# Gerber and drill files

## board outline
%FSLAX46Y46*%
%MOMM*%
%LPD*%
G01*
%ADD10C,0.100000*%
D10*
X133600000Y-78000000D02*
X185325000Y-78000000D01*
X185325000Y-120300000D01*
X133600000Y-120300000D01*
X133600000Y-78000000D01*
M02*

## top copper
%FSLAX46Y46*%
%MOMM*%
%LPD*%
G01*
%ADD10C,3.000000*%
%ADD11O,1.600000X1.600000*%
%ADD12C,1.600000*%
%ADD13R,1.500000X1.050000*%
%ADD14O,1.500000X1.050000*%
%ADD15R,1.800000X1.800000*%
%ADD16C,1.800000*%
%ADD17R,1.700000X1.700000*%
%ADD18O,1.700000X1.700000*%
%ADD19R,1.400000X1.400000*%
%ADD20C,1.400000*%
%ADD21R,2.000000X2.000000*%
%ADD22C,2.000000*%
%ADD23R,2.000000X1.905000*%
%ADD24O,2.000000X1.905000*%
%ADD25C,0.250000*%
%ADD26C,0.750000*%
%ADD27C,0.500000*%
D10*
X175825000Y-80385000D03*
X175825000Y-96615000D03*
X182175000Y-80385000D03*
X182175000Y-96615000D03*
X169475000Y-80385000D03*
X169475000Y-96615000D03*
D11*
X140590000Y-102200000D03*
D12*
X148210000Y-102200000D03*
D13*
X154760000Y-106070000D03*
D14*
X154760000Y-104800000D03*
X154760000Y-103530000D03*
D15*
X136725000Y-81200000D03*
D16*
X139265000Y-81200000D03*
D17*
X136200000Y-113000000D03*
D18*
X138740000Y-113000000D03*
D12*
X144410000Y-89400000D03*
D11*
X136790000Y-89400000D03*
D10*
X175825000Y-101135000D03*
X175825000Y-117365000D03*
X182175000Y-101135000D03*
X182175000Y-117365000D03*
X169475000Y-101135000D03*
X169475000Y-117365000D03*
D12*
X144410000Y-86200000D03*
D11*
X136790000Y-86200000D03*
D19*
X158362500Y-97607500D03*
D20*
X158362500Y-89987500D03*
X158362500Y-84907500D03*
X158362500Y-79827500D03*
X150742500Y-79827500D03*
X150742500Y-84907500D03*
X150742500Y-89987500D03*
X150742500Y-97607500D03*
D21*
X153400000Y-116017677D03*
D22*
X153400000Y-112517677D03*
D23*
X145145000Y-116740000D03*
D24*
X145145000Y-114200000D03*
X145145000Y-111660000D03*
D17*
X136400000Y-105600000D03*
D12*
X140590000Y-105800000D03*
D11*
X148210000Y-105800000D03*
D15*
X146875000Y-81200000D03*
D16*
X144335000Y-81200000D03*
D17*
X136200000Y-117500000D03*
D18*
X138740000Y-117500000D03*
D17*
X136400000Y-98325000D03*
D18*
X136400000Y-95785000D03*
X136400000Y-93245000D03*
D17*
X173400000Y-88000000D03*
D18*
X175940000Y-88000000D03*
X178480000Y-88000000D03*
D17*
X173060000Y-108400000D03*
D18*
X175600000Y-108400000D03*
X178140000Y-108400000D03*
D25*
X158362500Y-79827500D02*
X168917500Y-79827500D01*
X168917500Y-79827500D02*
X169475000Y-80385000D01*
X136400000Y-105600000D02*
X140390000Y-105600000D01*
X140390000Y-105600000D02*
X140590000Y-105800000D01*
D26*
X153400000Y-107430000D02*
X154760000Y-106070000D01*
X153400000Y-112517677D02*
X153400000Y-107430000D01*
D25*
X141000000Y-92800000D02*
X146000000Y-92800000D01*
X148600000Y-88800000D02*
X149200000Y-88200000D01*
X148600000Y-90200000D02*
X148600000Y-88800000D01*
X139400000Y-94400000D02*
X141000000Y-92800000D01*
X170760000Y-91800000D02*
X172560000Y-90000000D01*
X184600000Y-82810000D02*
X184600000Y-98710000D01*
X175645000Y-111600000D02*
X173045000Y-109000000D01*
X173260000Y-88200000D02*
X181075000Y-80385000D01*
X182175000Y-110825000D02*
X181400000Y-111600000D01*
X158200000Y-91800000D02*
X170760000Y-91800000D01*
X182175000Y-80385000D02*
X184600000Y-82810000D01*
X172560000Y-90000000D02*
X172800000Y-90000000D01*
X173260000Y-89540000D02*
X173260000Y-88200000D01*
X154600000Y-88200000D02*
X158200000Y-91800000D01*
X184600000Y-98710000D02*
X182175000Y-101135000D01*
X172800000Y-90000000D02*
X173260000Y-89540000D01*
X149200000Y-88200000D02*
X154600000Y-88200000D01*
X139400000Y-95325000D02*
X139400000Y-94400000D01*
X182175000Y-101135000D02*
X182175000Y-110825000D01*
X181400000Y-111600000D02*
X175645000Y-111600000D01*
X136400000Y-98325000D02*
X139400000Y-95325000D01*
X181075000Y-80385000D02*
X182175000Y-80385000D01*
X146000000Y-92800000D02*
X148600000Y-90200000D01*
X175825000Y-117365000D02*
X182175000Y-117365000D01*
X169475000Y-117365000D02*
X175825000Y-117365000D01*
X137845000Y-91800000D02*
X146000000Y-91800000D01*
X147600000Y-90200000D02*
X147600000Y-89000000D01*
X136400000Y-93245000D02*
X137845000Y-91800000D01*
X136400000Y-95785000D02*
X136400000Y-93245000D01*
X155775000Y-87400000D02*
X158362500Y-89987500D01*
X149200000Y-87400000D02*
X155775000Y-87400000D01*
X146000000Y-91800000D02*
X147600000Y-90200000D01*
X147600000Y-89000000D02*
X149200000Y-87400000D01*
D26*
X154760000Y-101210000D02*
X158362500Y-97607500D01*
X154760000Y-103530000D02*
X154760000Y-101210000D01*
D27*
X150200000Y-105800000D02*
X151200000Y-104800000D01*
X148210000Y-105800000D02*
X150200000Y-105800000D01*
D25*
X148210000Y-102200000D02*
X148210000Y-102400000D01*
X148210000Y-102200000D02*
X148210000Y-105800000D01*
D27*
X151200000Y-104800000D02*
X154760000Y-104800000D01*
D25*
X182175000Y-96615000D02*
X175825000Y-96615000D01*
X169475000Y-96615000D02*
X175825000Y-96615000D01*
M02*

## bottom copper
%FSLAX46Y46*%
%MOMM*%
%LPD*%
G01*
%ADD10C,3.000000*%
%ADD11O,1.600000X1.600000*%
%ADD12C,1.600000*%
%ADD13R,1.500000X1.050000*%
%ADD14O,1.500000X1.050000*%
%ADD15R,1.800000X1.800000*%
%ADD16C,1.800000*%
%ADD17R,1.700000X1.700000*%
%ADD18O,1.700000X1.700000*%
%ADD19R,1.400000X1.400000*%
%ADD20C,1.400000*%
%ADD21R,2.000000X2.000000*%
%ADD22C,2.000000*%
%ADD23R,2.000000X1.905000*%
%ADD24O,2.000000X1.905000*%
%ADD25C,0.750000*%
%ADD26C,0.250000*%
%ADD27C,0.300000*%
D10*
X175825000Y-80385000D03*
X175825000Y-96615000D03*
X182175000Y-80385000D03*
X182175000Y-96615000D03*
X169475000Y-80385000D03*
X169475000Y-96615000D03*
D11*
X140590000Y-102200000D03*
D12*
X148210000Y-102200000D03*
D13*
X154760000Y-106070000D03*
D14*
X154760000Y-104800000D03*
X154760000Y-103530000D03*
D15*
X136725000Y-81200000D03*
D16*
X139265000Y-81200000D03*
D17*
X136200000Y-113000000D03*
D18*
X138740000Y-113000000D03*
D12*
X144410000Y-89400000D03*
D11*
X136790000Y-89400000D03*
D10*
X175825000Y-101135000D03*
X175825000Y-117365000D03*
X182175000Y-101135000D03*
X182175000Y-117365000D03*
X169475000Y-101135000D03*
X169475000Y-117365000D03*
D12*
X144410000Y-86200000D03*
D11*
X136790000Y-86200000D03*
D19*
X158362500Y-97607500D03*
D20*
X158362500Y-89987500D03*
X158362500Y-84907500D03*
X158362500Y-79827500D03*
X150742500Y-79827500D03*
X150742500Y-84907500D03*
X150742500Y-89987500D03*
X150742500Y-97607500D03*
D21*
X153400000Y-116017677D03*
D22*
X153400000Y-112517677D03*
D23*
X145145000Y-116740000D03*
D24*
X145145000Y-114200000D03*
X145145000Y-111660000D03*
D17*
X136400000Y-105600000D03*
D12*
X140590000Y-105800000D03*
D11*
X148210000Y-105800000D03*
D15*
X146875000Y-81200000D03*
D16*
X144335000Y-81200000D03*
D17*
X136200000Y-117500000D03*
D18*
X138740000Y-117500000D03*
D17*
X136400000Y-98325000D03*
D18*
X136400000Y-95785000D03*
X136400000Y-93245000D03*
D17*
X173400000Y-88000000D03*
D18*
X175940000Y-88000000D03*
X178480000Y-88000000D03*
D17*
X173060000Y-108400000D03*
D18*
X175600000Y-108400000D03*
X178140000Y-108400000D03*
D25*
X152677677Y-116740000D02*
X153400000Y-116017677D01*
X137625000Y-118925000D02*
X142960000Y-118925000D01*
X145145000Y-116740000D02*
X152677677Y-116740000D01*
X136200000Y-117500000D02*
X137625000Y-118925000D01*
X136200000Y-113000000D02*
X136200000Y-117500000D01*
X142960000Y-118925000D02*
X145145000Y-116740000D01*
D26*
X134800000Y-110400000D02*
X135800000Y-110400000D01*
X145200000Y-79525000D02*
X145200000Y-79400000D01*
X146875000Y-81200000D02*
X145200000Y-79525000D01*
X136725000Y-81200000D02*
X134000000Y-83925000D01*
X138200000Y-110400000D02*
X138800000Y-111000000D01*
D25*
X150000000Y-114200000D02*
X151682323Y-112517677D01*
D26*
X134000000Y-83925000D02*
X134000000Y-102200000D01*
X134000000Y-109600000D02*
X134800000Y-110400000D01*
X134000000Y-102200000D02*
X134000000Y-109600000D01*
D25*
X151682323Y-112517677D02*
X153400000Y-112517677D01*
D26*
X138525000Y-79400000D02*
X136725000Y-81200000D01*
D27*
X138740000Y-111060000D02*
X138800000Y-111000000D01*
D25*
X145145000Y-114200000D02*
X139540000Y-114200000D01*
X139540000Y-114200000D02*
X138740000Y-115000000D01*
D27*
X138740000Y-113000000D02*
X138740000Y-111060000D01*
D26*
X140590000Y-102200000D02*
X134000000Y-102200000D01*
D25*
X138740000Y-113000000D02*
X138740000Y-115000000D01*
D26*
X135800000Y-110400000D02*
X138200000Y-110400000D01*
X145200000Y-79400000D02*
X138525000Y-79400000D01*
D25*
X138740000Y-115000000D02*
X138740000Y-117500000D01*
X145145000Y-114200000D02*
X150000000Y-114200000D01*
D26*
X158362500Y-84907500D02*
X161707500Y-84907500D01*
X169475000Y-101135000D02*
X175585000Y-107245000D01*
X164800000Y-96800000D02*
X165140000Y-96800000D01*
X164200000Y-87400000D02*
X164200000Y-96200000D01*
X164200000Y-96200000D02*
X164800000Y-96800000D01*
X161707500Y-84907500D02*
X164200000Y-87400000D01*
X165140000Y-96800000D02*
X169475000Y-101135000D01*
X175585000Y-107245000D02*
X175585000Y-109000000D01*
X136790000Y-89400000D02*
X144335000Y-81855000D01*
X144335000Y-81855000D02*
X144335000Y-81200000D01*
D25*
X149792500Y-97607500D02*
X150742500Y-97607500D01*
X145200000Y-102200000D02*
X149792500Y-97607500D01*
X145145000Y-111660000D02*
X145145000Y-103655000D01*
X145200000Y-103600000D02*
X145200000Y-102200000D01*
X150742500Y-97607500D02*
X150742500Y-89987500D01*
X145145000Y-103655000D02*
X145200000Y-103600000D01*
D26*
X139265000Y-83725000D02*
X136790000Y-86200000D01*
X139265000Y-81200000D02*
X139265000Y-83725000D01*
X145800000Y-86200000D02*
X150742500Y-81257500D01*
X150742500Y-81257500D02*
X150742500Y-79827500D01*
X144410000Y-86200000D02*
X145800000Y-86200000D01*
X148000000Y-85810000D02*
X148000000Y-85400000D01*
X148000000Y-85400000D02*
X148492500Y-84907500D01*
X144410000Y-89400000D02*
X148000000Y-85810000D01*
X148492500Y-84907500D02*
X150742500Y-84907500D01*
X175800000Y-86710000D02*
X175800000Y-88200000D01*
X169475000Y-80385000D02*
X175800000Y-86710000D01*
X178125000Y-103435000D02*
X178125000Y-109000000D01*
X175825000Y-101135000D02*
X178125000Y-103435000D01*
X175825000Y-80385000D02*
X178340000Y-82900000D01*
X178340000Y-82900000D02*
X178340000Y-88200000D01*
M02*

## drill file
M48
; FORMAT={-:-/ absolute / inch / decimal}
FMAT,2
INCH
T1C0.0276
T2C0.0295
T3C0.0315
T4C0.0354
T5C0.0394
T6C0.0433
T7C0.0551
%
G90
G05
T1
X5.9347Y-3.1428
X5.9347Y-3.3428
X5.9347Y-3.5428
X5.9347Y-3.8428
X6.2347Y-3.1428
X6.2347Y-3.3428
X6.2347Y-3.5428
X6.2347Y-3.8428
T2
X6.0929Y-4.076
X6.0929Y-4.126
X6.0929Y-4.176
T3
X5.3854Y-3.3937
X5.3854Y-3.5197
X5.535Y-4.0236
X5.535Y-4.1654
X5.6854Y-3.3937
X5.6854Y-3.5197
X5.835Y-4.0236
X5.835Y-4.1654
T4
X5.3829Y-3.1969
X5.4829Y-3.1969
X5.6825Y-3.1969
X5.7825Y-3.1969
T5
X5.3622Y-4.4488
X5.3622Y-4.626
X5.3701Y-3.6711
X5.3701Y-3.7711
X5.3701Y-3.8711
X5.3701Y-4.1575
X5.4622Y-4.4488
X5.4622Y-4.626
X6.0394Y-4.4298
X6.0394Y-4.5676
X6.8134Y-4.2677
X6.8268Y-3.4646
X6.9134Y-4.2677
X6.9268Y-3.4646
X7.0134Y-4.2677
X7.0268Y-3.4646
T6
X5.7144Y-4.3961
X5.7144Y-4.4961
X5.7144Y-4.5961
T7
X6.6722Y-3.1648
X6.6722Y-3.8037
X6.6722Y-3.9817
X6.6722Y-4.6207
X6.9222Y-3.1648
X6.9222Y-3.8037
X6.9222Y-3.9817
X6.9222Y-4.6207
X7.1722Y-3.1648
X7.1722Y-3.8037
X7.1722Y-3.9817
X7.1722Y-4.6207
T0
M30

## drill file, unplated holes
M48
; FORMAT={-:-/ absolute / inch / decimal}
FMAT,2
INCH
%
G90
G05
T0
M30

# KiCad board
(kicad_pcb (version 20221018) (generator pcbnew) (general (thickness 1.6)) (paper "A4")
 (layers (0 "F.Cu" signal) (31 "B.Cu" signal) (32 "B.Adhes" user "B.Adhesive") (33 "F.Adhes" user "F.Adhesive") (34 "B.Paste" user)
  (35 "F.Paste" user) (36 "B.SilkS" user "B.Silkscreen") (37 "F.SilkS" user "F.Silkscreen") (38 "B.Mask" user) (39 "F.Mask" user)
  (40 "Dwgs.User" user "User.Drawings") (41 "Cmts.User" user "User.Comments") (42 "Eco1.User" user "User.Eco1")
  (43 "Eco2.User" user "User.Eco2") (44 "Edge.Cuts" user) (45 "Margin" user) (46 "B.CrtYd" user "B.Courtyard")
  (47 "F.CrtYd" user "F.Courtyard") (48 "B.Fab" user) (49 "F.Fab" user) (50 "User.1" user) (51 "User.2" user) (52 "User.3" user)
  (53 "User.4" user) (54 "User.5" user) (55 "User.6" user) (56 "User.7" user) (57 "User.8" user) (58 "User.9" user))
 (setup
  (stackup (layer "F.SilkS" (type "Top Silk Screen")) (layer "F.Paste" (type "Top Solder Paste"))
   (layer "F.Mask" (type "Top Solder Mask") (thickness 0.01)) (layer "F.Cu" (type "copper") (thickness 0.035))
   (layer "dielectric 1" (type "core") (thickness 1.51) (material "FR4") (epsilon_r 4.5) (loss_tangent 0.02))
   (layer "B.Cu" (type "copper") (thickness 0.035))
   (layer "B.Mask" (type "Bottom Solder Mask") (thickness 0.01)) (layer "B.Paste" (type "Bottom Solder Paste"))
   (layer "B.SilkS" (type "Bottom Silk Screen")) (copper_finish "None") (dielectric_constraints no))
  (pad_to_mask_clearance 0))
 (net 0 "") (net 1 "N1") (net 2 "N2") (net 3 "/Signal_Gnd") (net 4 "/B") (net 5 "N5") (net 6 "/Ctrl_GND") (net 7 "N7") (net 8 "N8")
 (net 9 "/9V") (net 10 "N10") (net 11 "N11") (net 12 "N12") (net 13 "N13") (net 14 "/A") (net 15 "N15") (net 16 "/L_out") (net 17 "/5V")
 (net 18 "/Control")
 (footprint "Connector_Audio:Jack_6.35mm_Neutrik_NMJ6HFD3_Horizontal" (layer "F.Cu") (at 169.475 80.385)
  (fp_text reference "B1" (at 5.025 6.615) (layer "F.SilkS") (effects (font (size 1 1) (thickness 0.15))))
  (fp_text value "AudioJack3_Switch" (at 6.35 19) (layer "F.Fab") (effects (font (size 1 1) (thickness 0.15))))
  (pad "R" thru_hole circle (at 6.35 0) (size 3 3) (drill 1.4) (layers "*.Cu" "*.Mask") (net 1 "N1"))
  (pad "RN" thru_hole circle (at 6.35 16.23) (size 3 3) (drill 1.4) (layers "*.Cu" "*.Mask") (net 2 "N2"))
  (pad "S" thru_hole circle (at 12.7 0) (size 3 3) (drill 1.4) (layers "*.Cu" "*.Mask") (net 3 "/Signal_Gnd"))
  (pad "SN" thru_hole circle (at 12.7 16.23) (size 3 3) (drill 1.4) (layers "*.Cu" "*.Mask") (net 2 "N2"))
  (pad "T" thru_hole circle (at 0 0) (size 3 3) (drill 1.4) (layers "*.Cu" "*.Mask") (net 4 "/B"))
  (pad "TN" thru_hole circle (at 0 16.23) (size 3 3) (drill 1.4) (layers "*.Cu" "*.Mask") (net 2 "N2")))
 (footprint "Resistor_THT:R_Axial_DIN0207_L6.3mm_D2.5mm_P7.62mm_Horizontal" (layer "F.Cu") (at 148.21 102.2 180)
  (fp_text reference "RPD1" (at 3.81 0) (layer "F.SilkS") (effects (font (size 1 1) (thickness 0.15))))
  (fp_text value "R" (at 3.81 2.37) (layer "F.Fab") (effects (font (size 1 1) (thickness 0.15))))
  (pad "1" thru_hole circle (at 0 0 180) (size 1.6 1.6) (drill 0.8) (layers "*.Cu" "*.Mask") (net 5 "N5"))
  (pad "2" thru_hole oval (at 7.62 0 180) (size 1.6 1.6) (drill 0.8) (layers "*.Cu" "*.Mask") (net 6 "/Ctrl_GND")))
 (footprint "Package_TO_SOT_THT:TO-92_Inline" (layer "F.Cu") (at 154.76 106.07 90)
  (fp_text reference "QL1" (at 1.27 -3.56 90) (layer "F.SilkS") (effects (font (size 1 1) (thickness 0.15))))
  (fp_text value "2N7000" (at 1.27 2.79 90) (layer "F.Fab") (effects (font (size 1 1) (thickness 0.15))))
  (pad "1" thru_hole rect (at 0 0 90) (size 1.05 1.5) (drill 0.75) (layers "*.Cu" "*.Mask") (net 6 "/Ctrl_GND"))
  (pad "2" thru_hole oval (at 1.27 0 90) (size 1.05 1.5) (drill 0.75) (layers "*.Cu" "*.Mask") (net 5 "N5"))
  (pad "3" thru_hole oval (at 2.54 0 90) (size 1.05 1.5) (drill 0.75) (layers "*.Cu" "*.Mask") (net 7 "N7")))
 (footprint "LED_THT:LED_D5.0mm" (layer "F.Cu") (at 136.725 81.2)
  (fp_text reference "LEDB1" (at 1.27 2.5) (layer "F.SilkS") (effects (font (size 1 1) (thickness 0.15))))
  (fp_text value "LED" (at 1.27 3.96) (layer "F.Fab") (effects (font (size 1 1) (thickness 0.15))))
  (pad "1" thru_hole rect (at 0 0) (size 1.8 1.8) (drill 0.9) (layers "*.Cu" "*.Mask") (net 6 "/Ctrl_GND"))
  (pad "2" thru_hole circle (at 2.54 0) (size 1.8 1.8) (drill 0.9) (layers "*.Cu" "*.Mask") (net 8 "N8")))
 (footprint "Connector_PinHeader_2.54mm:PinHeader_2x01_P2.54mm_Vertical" (layer "F.Cu") (at 136.2 113)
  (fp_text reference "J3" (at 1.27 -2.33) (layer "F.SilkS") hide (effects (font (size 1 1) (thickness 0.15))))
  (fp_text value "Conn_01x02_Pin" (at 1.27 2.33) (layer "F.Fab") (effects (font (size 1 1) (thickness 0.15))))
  (pad "1" thru_hole rect (at 0 0) (size 1.7 1.7) (drill 1) (layers "*.Cu" "*.Mask") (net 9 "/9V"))
  (pad "2" thru_hole oval (at 2.54 0) (size 1.7 1.7) (drill 1) (layers "*.Cu" "*.Mask") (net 6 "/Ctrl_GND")))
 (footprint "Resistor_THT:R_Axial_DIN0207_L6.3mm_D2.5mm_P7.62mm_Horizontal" (layer "F.Cu") (at 144.41 89.4 180)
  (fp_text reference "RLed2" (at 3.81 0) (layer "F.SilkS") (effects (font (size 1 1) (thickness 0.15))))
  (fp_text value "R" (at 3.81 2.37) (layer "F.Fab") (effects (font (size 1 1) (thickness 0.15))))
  (pad "1" thru_hole circle (at 0 0 180) (size 1.6 1.6) (drill 0.8) (layers "*.Cu" "*.Mask") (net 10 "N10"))
  (pad "2" thru_hole oval (at 7.62 0 180) (size 1.6 1.6) (drill 0.8) (layers "*.Cu" "*.Mask") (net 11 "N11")))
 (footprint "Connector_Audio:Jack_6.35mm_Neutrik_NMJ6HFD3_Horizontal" (layer "F.Cu") (at 169.475 101.135)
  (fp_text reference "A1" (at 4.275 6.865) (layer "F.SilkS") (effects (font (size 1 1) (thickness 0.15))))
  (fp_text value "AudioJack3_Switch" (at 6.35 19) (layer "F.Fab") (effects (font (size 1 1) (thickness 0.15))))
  (pad "R" thru_hole circle (at 6.35 0) (size 3 3) (drill 1.4) (layers "*.Cu" "*.Mask") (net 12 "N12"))
  (pad "RN" thru_hole circle (at 6.35 16.23) (size 3 3) (drill 1.4) (layers "*.Cu" "*.Mask") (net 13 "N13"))
  (pad "S" thru_hole circle (at 12.7 0) (size 3 3) (drill 1.4) (layers "*.Cu" "*.Mask") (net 3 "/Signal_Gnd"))
  (pad "SN" thru_hole circle (at 12.7 16.23) (size 3 3) (drill 1.4) (layers "*.Cu" "*.Mask") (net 13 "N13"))
  (pad "T" thru_hole circle (at 0 0) (size 3 3) (drill 1.4) (layers "*.Cu" "*.Mask") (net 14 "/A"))
  (pad "TN" thru_hole circle (at 0 16.23) (size 3 3) (drill 1.4) (layers "*.Cu" "*.Mask") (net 13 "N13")))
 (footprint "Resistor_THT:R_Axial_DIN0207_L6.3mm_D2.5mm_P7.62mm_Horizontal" (layer "F.Cu") (at 144.41 86.2 180)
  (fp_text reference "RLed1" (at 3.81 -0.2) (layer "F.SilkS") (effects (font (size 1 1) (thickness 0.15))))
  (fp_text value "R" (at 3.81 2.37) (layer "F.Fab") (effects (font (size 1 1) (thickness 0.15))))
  (pad "1" thru_hole circle (at 0 0 180) (size 1.6 1.6) (drill 0.8) (layers "*.Cu" "*.Mask") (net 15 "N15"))
  (pad "2" thru_hole oval (at 7.62 0 180) (size 1.6 1.6) (drill 0.8) (layers "*.Cu" "*.Mask") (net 8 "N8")))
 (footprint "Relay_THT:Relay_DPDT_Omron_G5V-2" (layer "F.Cu") (at 158.3625 97.6075 180)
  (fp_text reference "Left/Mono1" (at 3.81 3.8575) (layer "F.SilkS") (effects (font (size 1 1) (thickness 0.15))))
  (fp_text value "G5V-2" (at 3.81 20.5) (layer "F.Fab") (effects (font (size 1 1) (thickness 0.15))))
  (pad "1" thru_hole rect (at 0 0 180) (size 1.4 1.4) (drill 0.7) (layers "*.Cu" "*.Mask") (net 7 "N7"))
  (pad "4" thru_hole circle (at 0 7.62 180) (size 1.4 1.4) (drill 0.7) (layers "*.Cu" "*.Mask") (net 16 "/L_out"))
  (pad "6" thru_hole circle (at 0 12.7 180) (size 1.4 1.4) (drill 0.7) (layers "*.Cu" "*.Mask") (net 14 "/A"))
  (pad "8" thru_hole circle (at 0 17.78 180) (size 1.4 1.4) (drill 0.7) (layers "*.Cu" "*.Mask") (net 4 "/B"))
  (pad "9" thru_hole circle (at 7.62 17.78 180) (size 1.4 1.4) (drill 0.7) (layers "*.Cu" "*.Mask") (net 15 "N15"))
  (pad "11" thru_hole circle (at 7.62 12.7 180) (size 1.4 1.4) (drill 0.7) (layers "*.Cu" "*.Mask") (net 10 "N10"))
  (pad "13" thru_hole circle (at 7.62 7.62 180) (size 1.4 1.4) (drill 0.7) (layers "*.Cu" "*.Mask") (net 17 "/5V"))
  (pad "16" thru_hole circle (at 7.62 0 180) (size 1.4 1.4) (drill 0.7) (layers "*.Cu" "*.Mask") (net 17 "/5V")))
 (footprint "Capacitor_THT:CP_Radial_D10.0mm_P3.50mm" (layer "F.Cu") (at 153.4 116.017677 90)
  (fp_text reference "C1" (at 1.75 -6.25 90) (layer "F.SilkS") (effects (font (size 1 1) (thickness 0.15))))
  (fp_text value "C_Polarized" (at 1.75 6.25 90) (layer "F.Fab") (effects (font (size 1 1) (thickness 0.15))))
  (pad "1" thru_hole rect (at 0 0 90) (size 2 2) (drill 1) (layers "*.Cu" "*.Mask") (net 9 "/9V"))
  (pad "2" thru_hole circle (at 3.5 0 90) (size 2 2) (drill 1) (layers "*.Cu" "*.Mask") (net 6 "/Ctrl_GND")))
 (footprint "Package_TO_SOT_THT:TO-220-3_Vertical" (layer "F.Cu") (at 145.145 116.74 90)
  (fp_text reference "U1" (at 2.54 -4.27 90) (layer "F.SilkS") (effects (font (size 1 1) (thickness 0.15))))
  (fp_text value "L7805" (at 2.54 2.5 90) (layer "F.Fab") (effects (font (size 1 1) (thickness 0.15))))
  (pad "1" thru_hole rect (at 0 0 90) (size 1.905 2) (drill 1.1) (layers "*.Cu" "*.Mask") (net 9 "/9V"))
  (pad "2" thru_hole oval (at 2.54 0 90) (size 1.905 2) (drill 1.1) (layers "*.Cu" "*.Mask") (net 6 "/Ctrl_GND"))
  (pad "3" thru_hole oval (at 5.08 0 90) (size 1.905 2) (drill 1.1) (layers "*.Cu" "*.Mask") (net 17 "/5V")))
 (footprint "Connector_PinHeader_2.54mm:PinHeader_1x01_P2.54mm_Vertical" (layer "F.Cu") (at 136.4 105.6 90)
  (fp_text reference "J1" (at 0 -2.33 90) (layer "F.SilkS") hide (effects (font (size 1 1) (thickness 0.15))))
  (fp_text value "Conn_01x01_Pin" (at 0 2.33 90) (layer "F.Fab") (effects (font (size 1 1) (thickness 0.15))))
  (pad "1" thru_hole rect (at 0 0 90) (size 1.7 1.7) (drill 1) (layers "*.Cu" "*.Mask") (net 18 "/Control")))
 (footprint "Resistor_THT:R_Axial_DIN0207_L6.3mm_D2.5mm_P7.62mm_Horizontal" (layer "F.Cu") (at 140.59 105.8)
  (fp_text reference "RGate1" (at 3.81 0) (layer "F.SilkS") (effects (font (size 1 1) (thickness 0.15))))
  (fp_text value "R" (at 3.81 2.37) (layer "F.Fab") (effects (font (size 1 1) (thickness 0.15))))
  (pad "1" thru_hole circle (at 0 0) (size 1.6 1.6) (drill 0.8) (layers "*.Cu" "*.Mask") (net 18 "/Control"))
  (pad "2" thru_hole oval (at 7.62 0) (size 1.6 1.6) (drill 0.8) (layers "*.Cu" "*.Mask") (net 5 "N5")))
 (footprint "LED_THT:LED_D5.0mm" (layer "F.Cu") (at 146.875 81.2 180)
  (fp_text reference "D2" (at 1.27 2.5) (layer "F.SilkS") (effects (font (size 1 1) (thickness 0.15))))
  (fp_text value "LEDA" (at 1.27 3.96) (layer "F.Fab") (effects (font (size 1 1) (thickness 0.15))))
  (pad "1" thru_hole rect (at 0 0 180) (size 1.8 1.8) (drill 0.9) (layers "*.Cu" "*.Mask") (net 6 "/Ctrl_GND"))
  (pad "2" thru_hole circle (at 2.54 0 180) (size 1.8 1.8) (drill 0.9) (layers "*.Cu" "*.Mask") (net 11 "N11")))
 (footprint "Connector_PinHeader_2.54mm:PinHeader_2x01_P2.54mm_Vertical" (layer "F.Cu") (at 136.2 117.5)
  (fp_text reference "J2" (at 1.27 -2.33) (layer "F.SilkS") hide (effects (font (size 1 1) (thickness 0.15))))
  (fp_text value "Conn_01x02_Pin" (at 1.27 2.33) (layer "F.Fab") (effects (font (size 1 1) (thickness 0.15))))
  (pad "1" thru_hole rect (at 0 0) (size 1.7 1.7) (drill 1) (layers "*.Cu" "*.Mask") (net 9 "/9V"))
  (pad "2" thru_hole oval (at 2.54 0) (size 1.7 1.7) (drill 1) (layers "*.Cu" "*.Mask") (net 6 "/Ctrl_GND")))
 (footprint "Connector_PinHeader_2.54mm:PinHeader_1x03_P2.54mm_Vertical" (layer "F.Cu") (at 136.4 98.325 180)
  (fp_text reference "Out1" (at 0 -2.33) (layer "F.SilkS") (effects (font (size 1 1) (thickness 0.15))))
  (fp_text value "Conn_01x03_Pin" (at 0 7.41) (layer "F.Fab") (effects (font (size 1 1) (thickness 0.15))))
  (pad "1" thru_hole rect (at 0 0 180) (size 1.7 1.7) (drill 1) (layers "*.Cu" "*.Mask") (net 3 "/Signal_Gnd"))
  (pad "2" thru_hole oval (at 0 2.54 180) (size 1.7 1.7) (drill 1) (layers "*.Cu" "*.Mask") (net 16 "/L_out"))
  (pad "3" thru_hole oval (at 0 5.08 180) (size 1.7 1.7) (drill 1) (layers "*.Cu" "*.Mask") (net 16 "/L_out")))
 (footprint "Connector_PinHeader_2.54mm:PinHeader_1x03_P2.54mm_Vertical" (layer "B.Cu") (at 173.4 88 -90)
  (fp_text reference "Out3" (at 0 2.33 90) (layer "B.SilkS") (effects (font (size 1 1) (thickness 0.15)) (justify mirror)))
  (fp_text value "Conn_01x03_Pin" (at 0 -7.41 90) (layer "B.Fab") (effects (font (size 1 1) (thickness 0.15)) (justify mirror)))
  (pad "1" thru_hole rect (at 0 0 270) (size 1.7 1.7) (drill 1) (layers "*.Cu" "*.Mask") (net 3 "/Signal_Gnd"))
  (pad "2" thru_hole oval (at 0 -2.54 270) (size 1.7 1.7) (drill 1) (layers "*.Cu" "*.Mask") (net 4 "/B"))
  (pad "3" thru_hole oval (at 0 -5.08 270) (size 1.7 1.7) (drill 1) (layers "*.Cu" "*.Mask") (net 1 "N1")))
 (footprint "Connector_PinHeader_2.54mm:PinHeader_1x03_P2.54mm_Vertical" (layer "B.Cu") (at 173.06 108.4 -90)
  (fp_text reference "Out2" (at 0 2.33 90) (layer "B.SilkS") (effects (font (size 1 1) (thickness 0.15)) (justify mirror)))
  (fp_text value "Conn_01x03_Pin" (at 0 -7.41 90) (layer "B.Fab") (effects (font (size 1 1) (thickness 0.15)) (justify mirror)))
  (pad "1" thru_hole rect (at 0 0 270) (size 1.7 1.7) (drill 1) (layers "*.Cu" "*.Mask") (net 3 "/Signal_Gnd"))
  (pad "2" thru_hole oval (at 0 -2.54 270) (size 1.7 1.7) (drill 1) (layers "*.Cu" "*.Mask") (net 14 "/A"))
  (pad "3" thru_hole oval (at 0 -5.08 270) (size 1.7 1.7) (drill 1) (layers "*.Cu" "*.Mask") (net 12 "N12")))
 (gr_rect (start 133.6 78) (end 185.325 120.3) (stroke (width 0.1) (type default)) (fill none) (layer "Edge.Cuts"))
 (segment (start 136.4 105.6) (end 140.39 105.6) (width 0.25) (layer "F.Cu") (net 18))
 (segment (start 140.39 105.6) (end 140.59 105.8) (width 0.25) (layer "F.Cu") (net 18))
 (segment (start 152.677677 116.74) (end 153.4 116.017677) (width 0.75) (layer "B.Cu") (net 9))
 (segment (start 137.625 118.925) (end 142.96 118.925) (width 0.75) (layer "B.Cu") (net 9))
 (segment (start 145.145 116.74) (end 152.677677 116.74) (width 0.75) (layer "B.Cu") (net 9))
 (segment (start 136.2 117.5) (end 137.625 118.925) (width 0.75) (layer "B.Cu") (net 9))
 (segment (start 136.2 113) (end 136.2 117.5) (width 0.75) (layer "B.Cu") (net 9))
 (segment (start 142.96 118.925) (end 145.145 116.74) (width 0.75) (layer "B.Cu") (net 9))
 (segment (start 153.4 107.43) (end 154.76 106.07) (width 0.75) (layer "F.Cu") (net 6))
 (segment (start 153.4 112.517677) (end 153.4 107.43) (width 0.75) (layer "F.Cu") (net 6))
 (segment (start 134.8 110.4) (end 135.8 110.4) (width 0.25) (layer "B.Cu") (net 6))
 (segment (start 145.2 79.525) (end 145.2 79.4) (width 0.25) (layer "B.Cu") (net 6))
 (segment (start 146.875 81.2) (end 145.2 79.525) (width 0.25) (layer "B.Cu") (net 6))
 (segment (start 136.725 81.2) (end 134 83.925) (width 0.25) (layer "B.Cu") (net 6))
 (segment (start 138.2 110.4) (end 138.8 111) (width 0.25) (layer "B.Cu") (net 6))
 (segment (start 150 114.2) (end 151.682323 112.517677) (width 0.75) (layer "B.Cu") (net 6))
 (segment (start 134 83.925) (end 134 102.2) (width 0.25) (layer "B.Cu") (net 6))
 (segment (start 134 109.6) (end 134.8 110.4) (width 0.25) (layer "B.Cu") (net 6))
 (segment (start 134 102.2) (end 134 109.6) (width 0.25) (layer "B.Cu") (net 6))
 (segment (start 151.682323 112.517677) (end 153.4 112.517677) (width 0.75) (layer "B.Cu") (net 6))
 (segment (start 138.525 79.4) (end 136.725 81.2) (width 0.25) (layer "B.Cu") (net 6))
 (segment (start 138.74 111.06) (end 138.8 111) (width 0.3) (layer "B.Cu") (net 6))
 (segment (start 145.145 114.2) (end 139.54 114.2) (width 0.75) (layer "B.Cu") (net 6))
 (segment (start 139.54 114.2) (end 138.74 115) (width 0.75) (layer "B.Cu") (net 6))
 (segment (start 138.74 113) (end 138.74 111.06) (width 0.3) (layer "B.Cu") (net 6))
 (segment (start 140.59 102.2) (end 134 102.2) (width 0.25) (layer "B.Cu") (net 6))
 (segment (start 138.74 113) (end 138.74 115) (width 0.75) (layer "B.Cu") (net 6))
 (segment (start 135.8 110.4) (end 138.2 110.4) (width 0.25) (layer "B.Cu") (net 6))
 (segment (start 145.2 79.4) (end 138.525 79.4) (width 0.25) (layer "B.Cu") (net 6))
 (segment (start 138.74 115) (end 138.74 117.5) (width 0.75) (layer "B.Cu") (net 6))
 (segment (start 145.145 114.2) (end 150 114.2) (width 0.75) (layer "B.Cu") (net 6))
 (segment (start 158.3625 84.9075) (end 161.7075 84.9075) (width 0.25) (layer "B.Cu") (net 14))
 (segment (start 169.475 101.135) (end 175.585 107.245) (width 0.25) (layer "B.Cu") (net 14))
 (segment (start 164.8 96.8) (end 165.14 96.8) (width 0.25) (layer "B.Cu") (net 14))
 (segment (start 164.2 87.4) (end 164.2 96.2) (width 0.25) (layer "B.Cu") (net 14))
 (segment (start 164.2 96.2) (end 164.8 96.8) (width 0.25) (layer "B.Cu") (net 14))
 (segment (start 161.7075 84.9075) (end 164.2 87.4) (width 0.25) (layer "B.Cu") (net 14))
 (segment (start 165.14 96.8) (end 169.475 101.135) (width 0.25) (layer "B.Cu") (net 14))
 (segment (start 175.585 107.245) (end 175.585 109) (width 0.25) (layer "B.Cu") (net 14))
 (segment (start 141 92.8) (end 146 92.8) (width 0.25) (layer "F.Cu") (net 3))
 (segment (start 148.6 88.8) (end 149.2 88.2) (width 0.25) (layer "F.Cu") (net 3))
 (segment (start 148.6 90.2) (end 148.6 88.8) (width 0.25) (layer "F.Cu") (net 3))
 (segment (start 139.4 94.4) (end 141 92.8) (width 0.25) (layer "F.Cu") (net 3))
 (segment (start 170.76 91.8) (end 172.56 90) (width 0.25) (layer "F.Cu") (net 3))
 (segment (start 184.6 82.81) (end 184.6 98.71) (width 0.25) (layer "F.Cu") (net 3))
 (segment (start 175.645 111.6) (end 173.045 109) (width 0.25) (layer "F.Cu") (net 3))
 (segment (start 173.26 88.2) (end 181.075 80.385) (width 0.25) (layer "F.Cu") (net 3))
 (segment (start 182.175 110.825) (end 181.4 111.6) (width 0.25) (layer "F.Cu") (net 3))
 (segment (start 158.2 91.8) (end 170.76 91.8) (width 0.25) (layer "F.Cu") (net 3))
 (segment (start 182.175 80.385) (end 184.6 82.81) (width 0.25) (layer "F.Cu") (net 3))
 (segment (start 172.56 90) (end 172.8 90) (width 0.25) (layer "F.Cu") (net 3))
 (segment (start 173.26 89.54) (end 173.26 88.2) (width 0.25) (layer "F.Cu") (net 3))
 (segment (start 154.6 88.2) (end 158.2 91.8) (width 0.25) (layer "F.Cu") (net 3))
 (segment (start 184.6 98.71) (end 182.175 101.135) (width 0.25) (layer "F.Cu") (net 3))
 (segment (start 172.8 90) (end 173.26 89.54) (width 0.25) (layer "F.Cu") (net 3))
 (segment (start 149.2 88.2) (end 154.6 88.2) (width 0.25) (layer "F.Cu") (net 3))
 (segment (start 139.4 95.325) (end 139.4 94.4) (width 0.25) (layer "F.Cu") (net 3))
 (segment (start 182.175 101.135) (end 182.175 110.825) (width 0.25) (layer "F.Cu") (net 3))
 (segment (start 181.4 111.6) (end 175.645 111.6) (width 0.25) (layer "F.Cu") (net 3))
 (segment (start 136.4 98.325) (end 139.4 95.325) (width 0.25) (layer "F.Cu") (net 3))
 (segment (start 181.075 80.385) (end 182.175 80.385) (width 0.25) (layer "F.Cu") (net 3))
 (segment (start 146 92.8) (end 148.6 90.2) (width 0.25) (layer "F.Cu") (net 3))
 (segment (start 175.825 117.365) (end 182.175 117.365) (width 0.25) (layer "F.Cu") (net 13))
 (segment (start 169.475 117.365) (end 175.825 117.365) (width 0.25) (layer "F.Cu") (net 13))
 (segment (start 168.9175 79.8275) (end 169.475 80.385) (width 0.25) (layer "F.Cu") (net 4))
 (segment (start 158.3625 79.8275) (end 168.9175 79.8275) (width 0.25) (layer "F.Cu") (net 4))
 (segment (start 175.8 86.71) (end 175.8 88.2) (width 0.25) (layer "B.Cu") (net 4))
 (segment (start 169.475 80.385) (end 175.8 86.71) (width 0.25) (layer "B.Cu") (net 4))
 (segment (start 136.79 89.4) (end 144.335 81.855) (width 0.25) (layer "B.Cu") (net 11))
 (segment (start 144.335 81.855) (end 144.335 81.2) (width 0.25) (layer "B.Cu") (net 11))
 (segment (start 149.7925 97.6075) (end 150.7425 97.6075) (width 0.75) (layer "B.Cu") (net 17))
 (segment (start 145.2 102.2) (end 149.7925 97.6075) (width 0.75) (layer "B.Cu") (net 17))
 (segment (start 145.145 111.66) (end 145.145 103.655) (width 0.75) (layer "B.Cu") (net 17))
 (segment (start 145.2 103.6) (end 145.2 102.2) (width 0.75) (layer "B.Cu") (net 17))
 (segment (start 150.7425 97.6075) (end 150.7425 89.9875) (width 0.75) (layer "B.Cu") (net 17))
 (segment (start 145.145 103.655) (end 145.2 103.6) (width 0.75) (layer "B.Cu") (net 17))
 (segment (start 137.845 91.8) (end 146 91.8) (width 0.25) (layer "F.Cu") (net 16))
 (segment (start 147.6 90.2) (end 147.6 89) (width 0.25) (layer "F.Cu") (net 16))
 (segment (start 136.4 93.245) (end 137.845 91.8) (width 0.25) (layer "F.Cu") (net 16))
 (segment (start 136.4 95.785) (end 136.4 93.245) (width 0.25) (layer "F.Cu") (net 16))
 (segment (start 155.775 87.4) (end 158.3625 89.9875) (width 0.25) (layer "F.Cu") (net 16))
 (segment (start 149.2 87.4) (end 155.775 87.4) (width 0.25) (layer "F.Cu") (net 16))
 (segment (start 146 91.8) (end 147.6 90.2) (width 0.25) (layer "F.Cu") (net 16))
 (segment (start 147.6 89) (end 149.2 87.4) (width 0.25) (layer "F.Cu") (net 16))
 (segment (start 139.265 83.725) (end 136.79 86.2) (width 0.25) (layer "B.Cu") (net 8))
 (segment (start 139.265 81.2) (end 139.265 83.725) (width 0.25) (layer "B.Cu") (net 8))
 (segment (start 145.8 86.2) (end 150.7425 81.2575) (width 0.25) (layer "B.Cu") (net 15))
 (segment (start 150.7425 81.2575) (end 150.7425 79.8275) (width 0.25) (layer "B.Cu") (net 15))
 (segment (start 144.41 86.2) (end 145.8 86.2) (width 0.25) (layer "B.Cu") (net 15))
 (segment (start 148 85.81) (end 148 85.4) (width 0.25) (layer "B.Cu") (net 10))
 (segment (start 148 85.4) (end 148.4925 84.9075) (width 0.25) (layer "B.Cu") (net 10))
 (segment (start 144.41 89.4) (end 148 85.81) (width 0.25) (layer "B.Cu") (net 10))
 (segment (start 148.4925 84.9075) (end 150.7425 84.9075) (width 0.25) (layer "B.Cu") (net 10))
 (segment (start 154.76 101.21) (end 158.3625 97.6075) (width 0.75) (layer "F.Cu") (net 7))
 (segment (start 154.76 103.53) (end 154.76 101.21) (width 0.75) (layer "F.Cu") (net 7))
 (segment (start 150.2 105.8) (end 151.2 104.8) (width 0.5) (layer "F.Cu") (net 5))
 (segment (start 148.21 105.8) (end 150.2 105.8) (width 0.5) (layer "F.Cu") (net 5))
 (segment (start 148.21 102.2) (end 148.21 102.4) (width 0.25) (layer "F.Cu") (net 5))
 (segment (start 148.21 102.2) (end 148.21 105.8) (width 0.25) (layer "F.Cu") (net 5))
 (segment (start 151.2 104.8) (end 154.76 104.8) (width 0.5) (layer "F.Cu") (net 5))
 (segment (start 182.175 96.615) (end 175.825 96.615) (width 0.25) (layer "F.Cu") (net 2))
 (segment (start 169.475 96.615) (end 175.825 96.615) (width 0.25) (layer "F.Cu") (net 2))
 (segment (start 178.125 103.435) (end 178.125 109) (width 0.25) (layer "B.Cu") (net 12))
 (segment (start 175.825 101.135) (end 178.125 103.435) (width 0.25) (layer "B.Cu") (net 12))
 (segment (start 175.825 80.385) (end 178.34 82.9) (width 0.25) (layer "B.Cu") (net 1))
 (segment (start 178.34 82.9) (end 178.34 88.2) (width 0.25) (layer "B.Cu") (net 1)))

